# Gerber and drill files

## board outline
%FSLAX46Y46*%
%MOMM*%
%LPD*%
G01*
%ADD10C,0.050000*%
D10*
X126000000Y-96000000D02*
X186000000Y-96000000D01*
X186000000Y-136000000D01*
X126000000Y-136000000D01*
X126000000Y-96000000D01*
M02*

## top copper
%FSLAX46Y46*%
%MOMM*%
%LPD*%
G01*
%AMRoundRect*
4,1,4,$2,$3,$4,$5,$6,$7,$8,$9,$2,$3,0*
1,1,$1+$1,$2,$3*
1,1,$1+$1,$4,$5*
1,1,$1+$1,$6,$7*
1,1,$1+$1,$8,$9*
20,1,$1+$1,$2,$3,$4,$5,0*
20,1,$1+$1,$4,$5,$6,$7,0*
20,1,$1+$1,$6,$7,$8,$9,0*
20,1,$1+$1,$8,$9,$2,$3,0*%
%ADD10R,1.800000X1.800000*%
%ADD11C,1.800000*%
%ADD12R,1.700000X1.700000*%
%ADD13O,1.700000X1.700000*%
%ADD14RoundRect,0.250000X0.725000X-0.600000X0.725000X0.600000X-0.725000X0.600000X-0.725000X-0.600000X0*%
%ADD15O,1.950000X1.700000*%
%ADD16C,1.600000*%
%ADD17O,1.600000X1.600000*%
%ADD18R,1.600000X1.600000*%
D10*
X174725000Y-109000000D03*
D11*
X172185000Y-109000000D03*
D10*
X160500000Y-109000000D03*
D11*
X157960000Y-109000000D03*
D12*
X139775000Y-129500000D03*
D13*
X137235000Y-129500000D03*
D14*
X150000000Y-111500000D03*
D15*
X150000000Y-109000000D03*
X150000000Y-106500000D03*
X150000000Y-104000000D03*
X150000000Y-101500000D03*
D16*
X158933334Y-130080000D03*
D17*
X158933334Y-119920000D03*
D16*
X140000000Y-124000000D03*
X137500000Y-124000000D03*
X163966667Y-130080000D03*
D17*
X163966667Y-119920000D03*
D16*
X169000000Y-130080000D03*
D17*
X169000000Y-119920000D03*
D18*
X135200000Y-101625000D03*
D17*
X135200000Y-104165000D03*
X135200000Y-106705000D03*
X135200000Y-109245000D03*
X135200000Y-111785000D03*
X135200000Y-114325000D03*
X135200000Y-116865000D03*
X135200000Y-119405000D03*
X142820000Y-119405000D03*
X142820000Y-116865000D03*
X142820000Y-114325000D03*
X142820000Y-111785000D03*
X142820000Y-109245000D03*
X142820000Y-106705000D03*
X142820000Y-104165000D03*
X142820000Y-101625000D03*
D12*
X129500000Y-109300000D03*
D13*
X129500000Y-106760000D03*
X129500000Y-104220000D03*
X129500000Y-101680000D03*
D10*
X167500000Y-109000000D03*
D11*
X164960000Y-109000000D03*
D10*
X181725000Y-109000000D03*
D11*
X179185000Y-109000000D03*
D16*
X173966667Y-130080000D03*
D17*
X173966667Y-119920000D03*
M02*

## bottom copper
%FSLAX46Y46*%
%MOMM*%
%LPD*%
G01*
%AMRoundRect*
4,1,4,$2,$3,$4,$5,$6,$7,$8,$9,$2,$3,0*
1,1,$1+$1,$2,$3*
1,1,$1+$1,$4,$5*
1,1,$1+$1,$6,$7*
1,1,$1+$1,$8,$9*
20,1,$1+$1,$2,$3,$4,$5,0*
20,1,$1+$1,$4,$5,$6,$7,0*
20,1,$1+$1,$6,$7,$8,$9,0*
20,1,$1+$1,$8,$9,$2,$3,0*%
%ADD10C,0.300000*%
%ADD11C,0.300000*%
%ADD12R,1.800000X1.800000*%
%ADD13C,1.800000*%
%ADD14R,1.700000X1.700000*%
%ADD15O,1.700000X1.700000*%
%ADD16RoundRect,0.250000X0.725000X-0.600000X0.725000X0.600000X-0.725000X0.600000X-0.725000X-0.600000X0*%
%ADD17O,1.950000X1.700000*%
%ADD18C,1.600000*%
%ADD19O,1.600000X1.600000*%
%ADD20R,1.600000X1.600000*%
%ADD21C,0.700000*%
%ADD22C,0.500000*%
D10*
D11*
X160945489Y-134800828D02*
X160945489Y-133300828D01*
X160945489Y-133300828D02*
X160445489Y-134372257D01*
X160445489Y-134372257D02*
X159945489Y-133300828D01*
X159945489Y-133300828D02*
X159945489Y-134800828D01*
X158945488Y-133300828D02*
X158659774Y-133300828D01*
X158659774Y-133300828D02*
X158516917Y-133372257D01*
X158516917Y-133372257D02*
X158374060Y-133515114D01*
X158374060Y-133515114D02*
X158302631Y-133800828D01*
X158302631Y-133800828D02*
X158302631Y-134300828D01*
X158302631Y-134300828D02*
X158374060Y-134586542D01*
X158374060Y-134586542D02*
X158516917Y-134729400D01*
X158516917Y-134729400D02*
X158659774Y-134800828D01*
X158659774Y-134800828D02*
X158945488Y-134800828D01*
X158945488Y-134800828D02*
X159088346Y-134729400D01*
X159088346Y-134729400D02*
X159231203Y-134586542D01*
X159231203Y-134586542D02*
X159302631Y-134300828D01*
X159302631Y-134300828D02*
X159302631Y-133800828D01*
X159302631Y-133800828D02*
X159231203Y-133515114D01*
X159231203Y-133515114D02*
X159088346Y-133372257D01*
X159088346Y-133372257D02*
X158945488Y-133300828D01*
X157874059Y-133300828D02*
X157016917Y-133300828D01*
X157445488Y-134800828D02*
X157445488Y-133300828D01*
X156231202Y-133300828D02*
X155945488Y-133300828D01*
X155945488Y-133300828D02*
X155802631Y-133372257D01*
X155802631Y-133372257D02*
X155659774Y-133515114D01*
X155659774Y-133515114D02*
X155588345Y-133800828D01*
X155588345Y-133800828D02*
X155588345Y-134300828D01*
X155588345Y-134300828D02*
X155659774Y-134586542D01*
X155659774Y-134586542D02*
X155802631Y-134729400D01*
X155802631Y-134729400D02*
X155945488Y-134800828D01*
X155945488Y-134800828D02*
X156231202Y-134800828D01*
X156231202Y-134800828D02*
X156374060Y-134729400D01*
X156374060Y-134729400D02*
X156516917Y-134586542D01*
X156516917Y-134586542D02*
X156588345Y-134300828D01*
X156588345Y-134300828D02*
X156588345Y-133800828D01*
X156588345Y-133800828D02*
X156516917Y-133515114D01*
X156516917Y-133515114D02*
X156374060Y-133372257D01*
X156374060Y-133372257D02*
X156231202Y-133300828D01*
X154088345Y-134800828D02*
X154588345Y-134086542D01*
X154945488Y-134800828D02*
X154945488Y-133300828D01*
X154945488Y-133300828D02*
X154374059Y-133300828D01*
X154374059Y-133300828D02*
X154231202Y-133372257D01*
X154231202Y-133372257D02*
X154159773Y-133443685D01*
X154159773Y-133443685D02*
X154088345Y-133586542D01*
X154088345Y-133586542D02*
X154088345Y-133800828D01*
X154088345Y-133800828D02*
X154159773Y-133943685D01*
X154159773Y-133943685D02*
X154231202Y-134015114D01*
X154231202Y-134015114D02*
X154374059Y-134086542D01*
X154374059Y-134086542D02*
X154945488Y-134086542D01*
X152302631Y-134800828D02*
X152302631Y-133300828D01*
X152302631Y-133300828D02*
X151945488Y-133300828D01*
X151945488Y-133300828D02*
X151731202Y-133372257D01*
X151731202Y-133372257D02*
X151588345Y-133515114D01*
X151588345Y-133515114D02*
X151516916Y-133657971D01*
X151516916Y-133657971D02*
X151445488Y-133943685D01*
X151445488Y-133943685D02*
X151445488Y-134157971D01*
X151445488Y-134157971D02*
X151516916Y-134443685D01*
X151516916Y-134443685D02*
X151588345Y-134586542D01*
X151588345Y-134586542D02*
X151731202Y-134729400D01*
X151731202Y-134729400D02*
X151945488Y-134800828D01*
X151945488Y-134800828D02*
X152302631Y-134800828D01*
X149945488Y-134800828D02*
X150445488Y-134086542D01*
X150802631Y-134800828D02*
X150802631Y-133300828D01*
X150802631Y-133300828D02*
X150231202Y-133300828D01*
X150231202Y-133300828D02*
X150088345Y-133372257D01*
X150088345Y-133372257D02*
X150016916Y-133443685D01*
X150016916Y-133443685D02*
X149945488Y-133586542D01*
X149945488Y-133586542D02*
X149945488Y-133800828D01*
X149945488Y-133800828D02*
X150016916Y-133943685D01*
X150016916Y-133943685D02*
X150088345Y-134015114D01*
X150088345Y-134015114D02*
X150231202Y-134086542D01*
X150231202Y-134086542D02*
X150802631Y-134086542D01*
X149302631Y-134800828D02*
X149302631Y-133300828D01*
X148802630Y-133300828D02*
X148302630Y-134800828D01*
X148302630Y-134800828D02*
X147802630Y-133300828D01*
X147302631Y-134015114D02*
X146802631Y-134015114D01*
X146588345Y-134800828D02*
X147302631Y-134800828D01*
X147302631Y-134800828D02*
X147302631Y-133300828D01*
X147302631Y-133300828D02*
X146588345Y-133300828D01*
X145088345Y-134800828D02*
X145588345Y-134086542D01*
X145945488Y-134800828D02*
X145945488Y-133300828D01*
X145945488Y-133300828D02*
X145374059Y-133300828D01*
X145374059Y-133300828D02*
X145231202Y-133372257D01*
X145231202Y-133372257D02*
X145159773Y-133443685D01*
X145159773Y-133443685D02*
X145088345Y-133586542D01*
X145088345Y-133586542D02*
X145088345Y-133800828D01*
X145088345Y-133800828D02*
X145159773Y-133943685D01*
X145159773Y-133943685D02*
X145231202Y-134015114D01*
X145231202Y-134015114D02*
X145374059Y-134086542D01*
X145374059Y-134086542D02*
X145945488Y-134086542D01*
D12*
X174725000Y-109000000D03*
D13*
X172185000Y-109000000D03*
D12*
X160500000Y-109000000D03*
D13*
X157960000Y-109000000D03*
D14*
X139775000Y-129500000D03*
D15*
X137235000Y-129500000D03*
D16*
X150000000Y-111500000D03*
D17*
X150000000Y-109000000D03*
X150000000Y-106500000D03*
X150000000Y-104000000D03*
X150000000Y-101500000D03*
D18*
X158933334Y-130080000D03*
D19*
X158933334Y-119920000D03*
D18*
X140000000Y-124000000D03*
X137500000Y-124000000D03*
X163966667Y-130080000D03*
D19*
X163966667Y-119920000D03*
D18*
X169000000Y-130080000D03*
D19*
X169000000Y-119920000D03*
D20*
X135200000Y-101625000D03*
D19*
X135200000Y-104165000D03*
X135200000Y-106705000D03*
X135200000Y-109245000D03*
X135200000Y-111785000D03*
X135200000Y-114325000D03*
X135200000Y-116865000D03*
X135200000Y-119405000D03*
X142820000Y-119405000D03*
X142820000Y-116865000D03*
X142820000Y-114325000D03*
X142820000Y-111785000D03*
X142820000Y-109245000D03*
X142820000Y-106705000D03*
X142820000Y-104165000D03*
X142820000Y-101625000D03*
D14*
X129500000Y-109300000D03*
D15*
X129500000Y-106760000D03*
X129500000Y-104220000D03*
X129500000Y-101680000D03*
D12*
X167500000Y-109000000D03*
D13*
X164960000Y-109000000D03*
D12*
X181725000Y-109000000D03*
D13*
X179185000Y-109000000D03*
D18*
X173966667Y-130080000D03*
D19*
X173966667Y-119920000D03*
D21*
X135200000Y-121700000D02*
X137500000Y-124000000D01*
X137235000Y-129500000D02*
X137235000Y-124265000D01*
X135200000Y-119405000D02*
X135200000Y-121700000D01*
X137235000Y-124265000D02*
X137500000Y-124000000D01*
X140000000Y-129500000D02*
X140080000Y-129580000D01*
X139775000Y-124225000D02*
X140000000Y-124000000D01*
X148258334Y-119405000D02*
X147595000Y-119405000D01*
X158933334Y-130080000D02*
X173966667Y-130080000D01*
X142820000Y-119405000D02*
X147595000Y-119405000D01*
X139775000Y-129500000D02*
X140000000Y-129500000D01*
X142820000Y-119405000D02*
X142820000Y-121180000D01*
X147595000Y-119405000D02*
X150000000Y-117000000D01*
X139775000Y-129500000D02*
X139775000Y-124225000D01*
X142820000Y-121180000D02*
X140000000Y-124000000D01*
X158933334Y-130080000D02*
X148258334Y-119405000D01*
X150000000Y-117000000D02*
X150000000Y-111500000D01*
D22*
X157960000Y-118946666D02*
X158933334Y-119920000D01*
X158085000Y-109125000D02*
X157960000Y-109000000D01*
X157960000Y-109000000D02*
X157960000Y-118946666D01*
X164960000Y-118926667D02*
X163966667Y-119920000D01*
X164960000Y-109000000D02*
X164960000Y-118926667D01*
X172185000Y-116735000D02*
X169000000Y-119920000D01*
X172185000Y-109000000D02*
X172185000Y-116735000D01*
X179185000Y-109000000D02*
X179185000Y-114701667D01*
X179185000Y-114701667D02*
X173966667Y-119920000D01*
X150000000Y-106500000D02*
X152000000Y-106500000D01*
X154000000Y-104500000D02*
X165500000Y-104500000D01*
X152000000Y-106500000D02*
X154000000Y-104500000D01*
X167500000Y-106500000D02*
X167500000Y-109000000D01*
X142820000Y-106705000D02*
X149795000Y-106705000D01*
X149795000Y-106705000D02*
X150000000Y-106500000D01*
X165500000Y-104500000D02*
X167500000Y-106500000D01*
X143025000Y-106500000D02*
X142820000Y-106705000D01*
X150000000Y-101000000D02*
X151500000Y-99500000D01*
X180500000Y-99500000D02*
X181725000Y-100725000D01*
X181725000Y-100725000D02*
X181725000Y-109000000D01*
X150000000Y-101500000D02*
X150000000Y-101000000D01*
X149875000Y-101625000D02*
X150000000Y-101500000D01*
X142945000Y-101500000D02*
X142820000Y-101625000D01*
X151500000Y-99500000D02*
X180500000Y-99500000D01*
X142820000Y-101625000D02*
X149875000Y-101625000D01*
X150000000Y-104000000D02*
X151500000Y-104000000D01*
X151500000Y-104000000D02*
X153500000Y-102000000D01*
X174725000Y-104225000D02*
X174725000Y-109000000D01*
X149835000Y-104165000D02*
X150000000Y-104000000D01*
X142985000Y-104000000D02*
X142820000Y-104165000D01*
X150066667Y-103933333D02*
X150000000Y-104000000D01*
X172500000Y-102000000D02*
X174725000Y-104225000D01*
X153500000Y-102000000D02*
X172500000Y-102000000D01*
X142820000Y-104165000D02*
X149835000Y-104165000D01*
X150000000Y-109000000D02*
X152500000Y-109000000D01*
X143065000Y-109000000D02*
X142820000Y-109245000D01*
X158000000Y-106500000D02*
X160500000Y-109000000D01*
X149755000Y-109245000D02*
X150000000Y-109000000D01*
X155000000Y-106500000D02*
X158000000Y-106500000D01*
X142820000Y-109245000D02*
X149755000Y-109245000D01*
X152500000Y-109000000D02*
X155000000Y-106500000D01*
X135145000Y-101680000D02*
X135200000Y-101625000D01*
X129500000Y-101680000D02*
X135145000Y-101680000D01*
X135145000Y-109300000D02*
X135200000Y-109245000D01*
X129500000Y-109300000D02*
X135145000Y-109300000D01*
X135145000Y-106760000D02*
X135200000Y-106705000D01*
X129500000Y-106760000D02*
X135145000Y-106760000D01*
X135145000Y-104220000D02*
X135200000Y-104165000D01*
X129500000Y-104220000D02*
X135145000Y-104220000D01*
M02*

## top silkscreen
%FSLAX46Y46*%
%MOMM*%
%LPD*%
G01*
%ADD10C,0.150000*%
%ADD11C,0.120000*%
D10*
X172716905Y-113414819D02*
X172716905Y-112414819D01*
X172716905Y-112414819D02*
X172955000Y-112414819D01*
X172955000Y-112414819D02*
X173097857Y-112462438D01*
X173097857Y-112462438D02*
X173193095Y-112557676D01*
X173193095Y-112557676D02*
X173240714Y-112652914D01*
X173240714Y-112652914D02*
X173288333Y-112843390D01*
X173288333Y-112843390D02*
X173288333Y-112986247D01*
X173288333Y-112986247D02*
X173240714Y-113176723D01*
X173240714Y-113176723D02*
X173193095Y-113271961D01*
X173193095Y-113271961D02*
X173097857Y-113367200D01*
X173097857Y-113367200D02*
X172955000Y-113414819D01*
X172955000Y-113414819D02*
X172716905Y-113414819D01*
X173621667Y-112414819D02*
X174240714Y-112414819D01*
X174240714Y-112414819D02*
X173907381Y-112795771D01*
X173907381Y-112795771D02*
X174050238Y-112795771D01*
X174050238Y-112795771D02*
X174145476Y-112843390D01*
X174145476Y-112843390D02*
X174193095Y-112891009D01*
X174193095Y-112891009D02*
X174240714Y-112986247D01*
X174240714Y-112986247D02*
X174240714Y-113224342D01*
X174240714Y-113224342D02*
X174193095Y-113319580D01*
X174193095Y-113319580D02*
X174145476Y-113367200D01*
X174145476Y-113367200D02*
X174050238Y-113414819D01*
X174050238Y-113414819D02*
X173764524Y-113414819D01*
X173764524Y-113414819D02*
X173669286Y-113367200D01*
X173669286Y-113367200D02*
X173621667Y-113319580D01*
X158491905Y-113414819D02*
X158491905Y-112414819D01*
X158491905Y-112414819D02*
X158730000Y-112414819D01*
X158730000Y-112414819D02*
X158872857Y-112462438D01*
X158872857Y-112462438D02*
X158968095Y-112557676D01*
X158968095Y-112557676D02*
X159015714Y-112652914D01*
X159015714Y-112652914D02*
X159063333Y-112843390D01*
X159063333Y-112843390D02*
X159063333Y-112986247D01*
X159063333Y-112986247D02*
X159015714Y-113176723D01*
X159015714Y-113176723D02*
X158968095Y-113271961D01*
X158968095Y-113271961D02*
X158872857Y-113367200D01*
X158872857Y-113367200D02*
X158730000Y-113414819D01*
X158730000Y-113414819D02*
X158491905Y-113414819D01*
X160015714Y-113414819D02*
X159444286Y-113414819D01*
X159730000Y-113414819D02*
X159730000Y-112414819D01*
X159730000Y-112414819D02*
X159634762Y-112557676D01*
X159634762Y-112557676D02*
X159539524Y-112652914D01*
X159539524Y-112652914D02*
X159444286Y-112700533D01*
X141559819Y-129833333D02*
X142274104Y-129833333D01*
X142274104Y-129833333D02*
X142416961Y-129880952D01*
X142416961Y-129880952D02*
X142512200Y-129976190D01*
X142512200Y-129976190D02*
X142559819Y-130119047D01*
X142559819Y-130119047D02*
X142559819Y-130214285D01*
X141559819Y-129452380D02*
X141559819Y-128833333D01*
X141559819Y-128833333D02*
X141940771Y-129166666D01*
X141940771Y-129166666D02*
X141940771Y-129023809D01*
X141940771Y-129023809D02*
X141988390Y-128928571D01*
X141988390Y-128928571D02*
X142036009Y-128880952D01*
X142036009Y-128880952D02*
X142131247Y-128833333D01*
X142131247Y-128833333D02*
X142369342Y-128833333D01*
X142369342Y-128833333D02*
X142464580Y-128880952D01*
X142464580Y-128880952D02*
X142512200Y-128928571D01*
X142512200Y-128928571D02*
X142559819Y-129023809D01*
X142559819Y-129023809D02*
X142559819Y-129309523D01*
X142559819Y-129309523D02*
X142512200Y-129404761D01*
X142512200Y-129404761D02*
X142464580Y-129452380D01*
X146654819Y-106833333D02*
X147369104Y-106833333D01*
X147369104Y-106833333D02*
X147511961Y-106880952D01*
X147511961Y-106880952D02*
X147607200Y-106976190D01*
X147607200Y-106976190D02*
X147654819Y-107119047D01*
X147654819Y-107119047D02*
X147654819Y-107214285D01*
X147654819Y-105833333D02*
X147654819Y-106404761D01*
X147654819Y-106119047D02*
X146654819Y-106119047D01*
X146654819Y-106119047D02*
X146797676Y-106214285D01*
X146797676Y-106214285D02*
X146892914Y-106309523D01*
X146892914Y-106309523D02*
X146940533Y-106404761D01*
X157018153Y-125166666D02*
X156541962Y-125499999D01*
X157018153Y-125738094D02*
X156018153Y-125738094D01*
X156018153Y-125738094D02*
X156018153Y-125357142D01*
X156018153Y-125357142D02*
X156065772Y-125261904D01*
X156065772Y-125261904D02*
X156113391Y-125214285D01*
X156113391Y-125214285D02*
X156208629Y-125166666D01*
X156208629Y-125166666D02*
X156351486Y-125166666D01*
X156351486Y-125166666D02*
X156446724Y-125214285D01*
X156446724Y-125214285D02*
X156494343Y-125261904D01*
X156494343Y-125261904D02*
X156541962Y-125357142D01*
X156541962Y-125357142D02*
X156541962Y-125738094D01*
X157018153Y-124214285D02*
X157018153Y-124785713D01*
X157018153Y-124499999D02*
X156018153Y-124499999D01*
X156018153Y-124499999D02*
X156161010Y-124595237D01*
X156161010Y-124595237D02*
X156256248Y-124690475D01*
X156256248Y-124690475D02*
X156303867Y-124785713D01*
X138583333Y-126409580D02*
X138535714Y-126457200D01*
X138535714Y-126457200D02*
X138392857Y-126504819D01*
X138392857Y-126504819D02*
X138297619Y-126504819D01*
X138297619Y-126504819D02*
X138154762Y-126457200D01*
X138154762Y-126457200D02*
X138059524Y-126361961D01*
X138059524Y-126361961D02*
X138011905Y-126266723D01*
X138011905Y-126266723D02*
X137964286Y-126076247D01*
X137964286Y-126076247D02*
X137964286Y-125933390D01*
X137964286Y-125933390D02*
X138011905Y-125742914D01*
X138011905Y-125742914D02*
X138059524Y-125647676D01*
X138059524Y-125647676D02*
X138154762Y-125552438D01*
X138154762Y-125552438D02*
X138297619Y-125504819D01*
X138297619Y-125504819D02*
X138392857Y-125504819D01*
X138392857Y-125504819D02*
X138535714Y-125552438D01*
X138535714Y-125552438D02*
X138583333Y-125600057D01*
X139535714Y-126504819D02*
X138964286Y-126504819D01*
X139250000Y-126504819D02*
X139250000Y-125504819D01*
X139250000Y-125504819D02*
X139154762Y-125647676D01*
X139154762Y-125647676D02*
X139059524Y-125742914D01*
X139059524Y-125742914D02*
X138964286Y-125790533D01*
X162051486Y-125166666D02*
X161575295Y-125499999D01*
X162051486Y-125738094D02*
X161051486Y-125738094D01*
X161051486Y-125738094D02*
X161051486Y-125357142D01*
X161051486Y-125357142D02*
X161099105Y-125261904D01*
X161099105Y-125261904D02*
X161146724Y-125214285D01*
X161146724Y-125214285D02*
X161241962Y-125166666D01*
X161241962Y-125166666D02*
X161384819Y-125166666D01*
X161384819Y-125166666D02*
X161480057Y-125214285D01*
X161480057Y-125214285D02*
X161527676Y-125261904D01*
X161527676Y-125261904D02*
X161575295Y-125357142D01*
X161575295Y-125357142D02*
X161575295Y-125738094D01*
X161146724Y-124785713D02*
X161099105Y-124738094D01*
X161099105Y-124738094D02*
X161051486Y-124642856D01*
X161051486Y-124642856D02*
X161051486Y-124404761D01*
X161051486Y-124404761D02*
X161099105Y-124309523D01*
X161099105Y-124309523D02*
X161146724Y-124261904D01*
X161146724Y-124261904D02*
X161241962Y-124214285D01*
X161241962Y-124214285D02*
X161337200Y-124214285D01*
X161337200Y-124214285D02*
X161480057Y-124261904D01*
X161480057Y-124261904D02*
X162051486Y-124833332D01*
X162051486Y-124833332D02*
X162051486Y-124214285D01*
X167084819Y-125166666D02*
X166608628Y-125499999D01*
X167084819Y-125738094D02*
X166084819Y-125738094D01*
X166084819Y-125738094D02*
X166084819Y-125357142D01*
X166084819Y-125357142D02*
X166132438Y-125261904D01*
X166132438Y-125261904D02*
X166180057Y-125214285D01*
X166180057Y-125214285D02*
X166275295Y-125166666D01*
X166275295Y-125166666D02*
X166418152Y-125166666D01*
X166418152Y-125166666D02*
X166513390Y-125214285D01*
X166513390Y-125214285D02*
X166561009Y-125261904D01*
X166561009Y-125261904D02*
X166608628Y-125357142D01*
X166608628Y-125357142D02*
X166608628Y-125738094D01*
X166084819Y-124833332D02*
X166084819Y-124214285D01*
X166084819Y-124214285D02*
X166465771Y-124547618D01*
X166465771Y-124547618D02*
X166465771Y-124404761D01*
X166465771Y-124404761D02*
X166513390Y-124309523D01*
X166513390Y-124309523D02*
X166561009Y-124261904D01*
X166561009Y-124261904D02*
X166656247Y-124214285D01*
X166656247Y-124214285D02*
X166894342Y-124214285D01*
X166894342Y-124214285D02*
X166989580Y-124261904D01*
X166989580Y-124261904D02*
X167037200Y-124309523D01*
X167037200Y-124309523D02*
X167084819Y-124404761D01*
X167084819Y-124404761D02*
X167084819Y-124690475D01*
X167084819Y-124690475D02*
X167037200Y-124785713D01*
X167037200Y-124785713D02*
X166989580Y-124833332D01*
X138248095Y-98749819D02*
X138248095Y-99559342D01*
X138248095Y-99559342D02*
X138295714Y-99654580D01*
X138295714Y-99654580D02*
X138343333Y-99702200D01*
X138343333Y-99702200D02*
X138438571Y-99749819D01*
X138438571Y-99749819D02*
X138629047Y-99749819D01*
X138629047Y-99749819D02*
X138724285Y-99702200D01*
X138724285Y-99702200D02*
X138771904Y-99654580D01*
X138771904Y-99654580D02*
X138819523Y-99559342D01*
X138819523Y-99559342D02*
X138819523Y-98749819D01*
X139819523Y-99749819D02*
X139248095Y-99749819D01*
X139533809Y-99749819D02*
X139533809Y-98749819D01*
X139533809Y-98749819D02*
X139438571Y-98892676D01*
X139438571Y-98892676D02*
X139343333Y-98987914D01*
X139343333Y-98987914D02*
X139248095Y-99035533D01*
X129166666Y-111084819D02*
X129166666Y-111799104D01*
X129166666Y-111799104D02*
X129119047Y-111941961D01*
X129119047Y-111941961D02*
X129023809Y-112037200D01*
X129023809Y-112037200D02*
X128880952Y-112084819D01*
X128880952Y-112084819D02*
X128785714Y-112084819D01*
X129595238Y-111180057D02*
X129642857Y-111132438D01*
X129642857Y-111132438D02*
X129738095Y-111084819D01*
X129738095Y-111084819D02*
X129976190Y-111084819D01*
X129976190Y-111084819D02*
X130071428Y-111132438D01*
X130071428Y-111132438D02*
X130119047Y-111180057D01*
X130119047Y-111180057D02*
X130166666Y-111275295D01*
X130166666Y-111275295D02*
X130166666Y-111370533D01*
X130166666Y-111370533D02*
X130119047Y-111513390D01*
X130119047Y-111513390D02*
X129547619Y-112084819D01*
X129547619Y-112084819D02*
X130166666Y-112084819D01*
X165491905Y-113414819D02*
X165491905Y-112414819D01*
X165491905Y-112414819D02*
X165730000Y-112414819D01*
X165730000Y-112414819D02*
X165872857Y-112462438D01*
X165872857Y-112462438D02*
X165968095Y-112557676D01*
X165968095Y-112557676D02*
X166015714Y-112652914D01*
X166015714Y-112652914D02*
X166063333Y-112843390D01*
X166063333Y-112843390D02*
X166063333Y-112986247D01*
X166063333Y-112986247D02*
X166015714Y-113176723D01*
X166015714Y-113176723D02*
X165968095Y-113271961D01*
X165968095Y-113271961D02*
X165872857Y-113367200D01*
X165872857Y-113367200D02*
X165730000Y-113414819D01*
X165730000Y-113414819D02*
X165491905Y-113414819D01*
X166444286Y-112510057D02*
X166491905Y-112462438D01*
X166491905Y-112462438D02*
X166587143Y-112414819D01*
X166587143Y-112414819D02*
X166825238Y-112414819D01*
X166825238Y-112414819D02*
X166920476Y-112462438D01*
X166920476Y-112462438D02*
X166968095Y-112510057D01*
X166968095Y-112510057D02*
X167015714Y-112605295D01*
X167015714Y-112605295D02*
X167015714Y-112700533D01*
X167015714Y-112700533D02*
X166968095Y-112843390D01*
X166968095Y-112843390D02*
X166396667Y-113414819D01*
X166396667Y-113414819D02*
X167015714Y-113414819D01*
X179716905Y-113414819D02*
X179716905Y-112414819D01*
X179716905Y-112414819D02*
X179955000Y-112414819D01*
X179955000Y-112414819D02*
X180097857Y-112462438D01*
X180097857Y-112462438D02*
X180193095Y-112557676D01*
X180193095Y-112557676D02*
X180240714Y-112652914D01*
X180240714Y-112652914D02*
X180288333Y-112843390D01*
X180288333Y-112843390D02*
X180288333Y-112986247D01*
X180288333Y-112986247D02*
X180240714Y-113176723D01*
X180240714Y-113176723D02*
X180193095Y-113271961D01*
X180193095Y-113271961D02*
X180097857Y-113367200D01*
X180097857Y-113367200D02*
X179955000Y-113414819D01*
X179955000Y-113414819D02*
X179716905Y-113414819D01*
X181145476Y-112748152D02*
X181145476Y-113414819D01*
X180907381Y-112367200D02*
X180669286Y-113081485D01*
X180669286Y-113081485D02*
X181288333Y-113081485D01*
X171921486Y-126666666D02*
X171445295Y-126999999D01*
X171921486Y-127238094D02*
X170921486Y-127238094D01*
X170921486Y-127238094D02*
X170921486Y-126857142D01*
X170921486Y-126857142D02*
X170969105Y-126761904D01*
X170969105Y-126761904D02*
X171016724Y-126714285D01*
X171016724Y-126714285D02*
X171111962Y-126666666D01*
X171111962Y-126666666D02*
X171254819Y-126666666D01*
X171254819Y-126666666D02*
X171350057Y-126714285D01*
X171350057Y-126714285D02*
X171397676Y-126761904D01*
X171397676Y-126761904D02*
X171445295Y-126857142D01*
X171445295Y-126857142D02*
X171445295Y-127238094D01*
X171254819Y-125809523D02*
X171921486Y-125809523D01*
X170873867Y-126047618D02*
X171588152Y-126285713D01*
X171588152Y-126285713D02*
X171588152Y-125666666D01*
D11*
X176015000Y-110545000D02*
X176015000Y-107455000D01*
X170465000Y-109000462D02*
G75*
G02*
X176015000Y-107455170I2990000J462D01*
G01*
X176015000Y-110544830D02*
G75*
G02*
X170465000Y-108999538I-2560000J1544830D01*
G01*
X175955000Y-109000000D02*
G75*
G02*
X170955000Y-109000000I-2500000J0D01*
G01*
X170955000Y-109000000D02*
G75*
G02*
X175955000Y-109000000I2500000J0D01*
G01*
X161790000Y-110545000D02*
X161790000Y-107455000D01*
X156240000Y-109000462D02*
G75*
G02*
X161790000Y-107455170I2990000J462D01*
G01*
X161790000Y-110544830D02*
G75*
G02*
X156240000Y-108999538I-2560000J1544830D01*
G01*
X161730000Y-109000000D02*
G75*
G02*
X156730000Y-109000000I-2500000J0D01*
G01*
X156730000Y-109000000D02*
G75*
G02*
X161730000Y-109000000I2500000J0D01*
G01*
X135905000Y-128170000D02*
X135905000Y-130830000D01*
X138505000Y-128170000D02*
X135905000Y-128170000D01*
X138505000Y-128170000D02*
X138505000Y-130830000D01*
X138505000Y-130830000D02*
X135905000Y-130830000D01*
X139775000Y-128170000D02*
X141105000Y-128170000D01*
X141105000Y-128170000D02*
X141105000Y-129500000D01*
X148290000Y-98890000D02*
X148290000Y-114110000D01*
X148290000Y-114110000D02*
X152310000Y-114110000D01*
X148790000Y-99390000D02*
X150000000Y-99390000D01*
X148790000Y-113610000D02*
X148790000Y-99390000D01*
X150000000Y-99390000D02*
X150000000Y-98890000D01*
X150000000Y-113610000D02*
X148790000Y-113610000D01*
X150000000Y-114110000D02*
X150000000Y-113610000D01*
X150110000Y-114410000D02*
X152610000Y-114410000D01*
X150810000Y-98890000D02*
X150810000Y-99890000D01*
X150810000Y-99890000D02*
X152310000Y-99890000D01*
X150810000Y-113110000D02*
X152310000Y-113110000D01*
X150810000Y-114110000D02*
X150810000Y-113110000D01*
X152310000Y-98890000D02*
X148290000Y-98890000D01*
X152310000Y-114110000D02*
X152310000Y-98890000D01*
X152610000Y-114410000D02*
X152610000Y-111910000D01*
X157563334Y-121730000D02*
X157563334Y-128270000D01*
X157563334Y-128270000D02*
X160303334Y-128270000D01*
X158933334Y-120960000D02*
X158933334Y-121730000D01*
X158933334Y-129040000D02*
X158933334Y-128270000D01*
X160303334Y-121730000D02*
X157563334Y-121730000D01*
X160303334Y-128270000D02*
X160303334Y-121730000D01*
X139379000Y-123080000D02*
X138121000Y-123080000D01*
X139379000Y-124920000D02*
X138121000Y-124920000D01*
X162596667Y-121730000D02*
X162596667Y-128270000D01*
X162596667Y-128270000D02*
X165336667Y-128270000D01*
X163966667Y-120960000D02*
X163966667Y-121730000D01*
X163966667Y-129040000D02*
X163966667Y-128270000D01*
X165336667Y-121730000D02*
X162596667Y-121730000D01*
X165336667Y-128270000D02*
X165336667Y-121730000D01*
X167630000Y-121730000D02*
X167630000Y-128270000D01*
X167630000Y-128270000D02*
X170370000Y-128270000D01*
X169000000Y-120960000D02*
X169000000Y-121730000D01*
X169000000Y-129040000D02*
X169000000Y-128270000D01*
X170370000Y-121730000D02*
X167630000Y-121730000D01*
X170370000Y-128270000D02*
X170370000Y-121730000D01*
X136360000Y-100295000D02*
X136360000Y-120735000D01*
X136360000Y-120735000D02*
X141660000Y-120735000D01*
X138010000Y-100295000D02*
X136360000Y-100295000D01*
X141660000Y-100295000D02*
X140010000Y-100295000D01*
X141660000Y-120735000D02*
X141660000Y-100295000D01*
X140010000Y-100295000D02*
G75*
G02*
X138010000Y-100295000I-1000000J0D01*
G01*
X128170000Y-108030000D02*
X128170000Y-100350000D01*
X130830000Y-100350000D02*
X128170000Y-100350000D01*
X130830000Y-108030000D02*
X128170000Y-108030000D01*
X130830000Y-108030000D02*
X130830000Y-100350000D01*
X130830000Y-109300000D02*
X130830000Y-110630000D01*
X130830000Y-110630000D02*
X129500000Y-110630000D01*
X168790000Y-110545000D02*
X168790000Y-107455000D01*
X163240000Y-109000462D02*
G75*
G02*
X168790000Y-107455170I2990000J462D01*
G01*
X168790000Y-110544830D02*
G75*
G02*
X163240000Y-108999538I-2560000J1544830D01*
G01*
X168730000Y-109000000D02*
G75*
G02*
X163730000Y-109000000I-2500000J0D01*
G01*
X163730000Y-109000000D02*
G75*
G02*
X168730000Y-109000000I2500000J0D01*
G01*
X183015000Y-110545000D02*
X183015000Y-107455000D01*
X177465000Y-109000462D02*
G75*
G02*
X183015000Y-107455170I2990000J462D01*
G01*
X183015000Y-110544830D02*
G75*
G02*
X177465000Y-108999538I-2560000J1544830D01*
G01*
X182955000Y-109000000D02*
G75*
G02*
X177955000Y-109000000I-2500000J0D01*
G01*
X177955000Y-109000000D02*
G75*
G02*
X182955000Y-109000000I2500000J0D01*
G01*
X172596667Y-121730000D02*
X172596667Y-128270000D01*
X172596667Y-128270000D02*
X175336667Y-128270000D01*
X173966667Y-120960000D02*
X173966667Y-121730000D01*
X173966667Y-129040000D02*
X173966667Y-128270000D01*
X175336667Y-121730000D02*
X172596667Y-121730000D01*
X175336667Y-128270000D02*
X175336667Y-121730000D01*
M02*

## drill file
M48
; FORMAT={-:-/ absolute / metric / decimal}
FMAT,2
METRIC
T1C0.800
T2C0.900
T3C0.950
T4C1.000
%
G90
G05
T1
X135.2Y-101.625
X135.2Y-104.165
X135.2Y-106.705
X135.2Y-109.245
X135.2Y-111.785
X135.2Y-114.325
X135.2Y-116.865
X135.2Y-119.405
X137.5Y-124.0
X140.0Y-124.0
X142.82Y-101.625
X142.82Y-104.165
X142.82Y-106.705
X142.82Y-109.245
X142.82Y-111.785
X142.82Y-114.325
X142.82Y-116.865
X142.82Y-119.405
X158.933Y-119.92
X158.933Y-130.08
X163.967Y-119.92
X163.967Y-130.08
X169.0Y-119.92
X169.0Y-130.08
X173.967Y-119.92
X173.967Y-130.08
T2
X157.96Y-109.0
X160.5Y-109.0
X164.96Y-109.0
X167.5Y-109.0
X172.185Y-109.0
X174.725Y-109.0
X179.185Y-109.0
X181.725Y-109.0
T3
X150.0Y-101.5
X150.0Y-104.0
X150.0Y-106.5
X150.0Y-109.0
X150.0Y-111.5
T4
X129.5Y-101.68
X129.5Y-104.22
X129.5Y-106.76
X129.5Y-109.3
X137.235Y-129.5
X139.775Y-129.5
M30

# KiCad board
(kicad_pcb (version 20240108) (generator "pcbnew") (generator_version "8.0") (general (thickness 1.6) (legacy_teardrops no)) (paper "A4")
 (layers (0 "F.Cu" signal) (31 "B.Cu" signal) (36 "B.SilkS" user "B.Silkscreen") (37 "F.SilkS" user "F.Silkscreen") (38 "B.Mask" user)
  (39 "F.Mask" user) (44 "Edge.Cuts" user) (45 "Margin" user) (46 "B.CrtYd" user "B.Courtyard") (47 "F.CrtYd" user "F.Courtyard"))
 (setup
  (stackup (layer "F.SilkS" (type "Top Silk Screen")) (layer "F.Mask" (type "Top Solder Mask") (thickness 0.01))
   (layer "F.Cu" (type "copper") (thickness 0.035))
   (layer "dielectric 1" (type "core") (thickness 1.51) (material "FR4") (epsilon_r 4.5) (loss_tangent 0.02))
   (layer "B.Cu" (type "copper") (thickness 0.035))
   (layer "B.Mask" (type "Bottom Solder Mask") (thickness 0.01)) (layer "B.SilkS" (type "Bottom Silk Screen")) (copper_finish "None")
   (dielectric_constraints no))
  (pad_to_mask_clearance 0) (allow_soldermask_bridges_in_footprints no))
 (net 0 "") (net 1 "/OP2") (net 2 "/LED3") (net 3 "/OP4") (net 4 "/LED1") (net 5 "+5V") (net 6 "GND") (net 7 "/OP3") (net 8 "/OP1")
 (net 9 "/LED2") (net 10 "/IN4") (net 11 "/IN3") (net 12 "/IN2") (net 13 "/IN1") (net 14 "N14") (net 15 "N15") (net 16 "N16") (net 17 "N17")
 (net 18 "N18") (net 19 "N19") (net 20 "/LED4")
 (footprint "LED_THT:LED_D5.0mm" (layer "F.Cu") (at 174.725 109 180)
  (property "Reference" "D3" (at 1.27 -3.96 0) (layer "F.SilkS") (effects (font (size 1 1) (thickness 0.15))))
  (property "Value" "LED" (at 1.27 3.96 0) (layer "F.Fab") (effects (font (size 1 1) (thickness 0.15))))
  (fp_line (start -1.29 -1.545) (end -1.29 1.545) (stroke (width 0.12) (type solid)) (layer "F.SilkS"))
  (fp_arc (start 4.26 -0.000462) (mid 2.072002 2.880433) (end -1.29 1.54483) (stroke (width 0.12) (type solid)) (layer "F.SilkS"))
  (fp_arc (start -1.29 -1.54483) (mid 2.072002 -2.880433) (end 4.26 0.000462) (stroke (width 0.12) (type solid)) (layer "F.SilkS"))
  (fp_circle (center 1.27 0) (end 3.77 0) (stroke (width 0.12) (type solid)) (fill none) (layer "F.SilkS"))
  (pad "1" thru_hole rect (at 0 0 180) (size 1.8 1.8) (drill 0.9) (layers "*.Cu" "*.Mask") (remove_unused_layers no) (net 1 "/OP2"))
  (pad "2" thru_hole circle (at 2.54 0 180) (size 1.8 1.8) (drill 0.9) (layers "*.Cu" "*.Mask") (remove_unused_layers no) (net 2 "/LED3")))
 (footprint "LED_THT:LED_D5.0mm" (layer "F.Cu") (at 160.5 109 180)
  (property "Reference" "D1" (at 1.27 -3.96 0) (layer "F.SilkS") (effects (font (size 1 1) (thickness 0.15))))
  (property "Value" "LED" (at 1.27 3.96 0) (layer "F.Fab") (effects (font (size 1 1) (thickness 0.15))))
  (fp_line (start -1.29 -1.545) (end -1.29 1.545) (stroke (width 0.12) (type solid)) (layer "F.SilkS"))
  (fp_arc (start 4.26 -0.000462) (mid 2.072002 2.880433) (end -1.29 1.54483) (stroke (width 0.12) (type solid)) (layer "F.SilkS"))
  (fp_arc (start -1.29 -1.54483) (mid 2.072002 -2.880433) (end 4.26 0.000462) (stroke (width 0.12) (type solid)) (layer "F.SilkS"))
  (fp_circle (center 1.27 0) (end 3.77 0) (stroke (width 0.12) (type solid)) (fill none) (layer "F.SilkS"))
  (pad "1" thru_hole rect (at 0 0 180) (size 1.8 1.8) (drill 0.9) (layers "*.Cu" "*.Mask") (remove_unused_layers no) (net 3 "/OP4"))
  (pad "2" thru_hole circle (at 2.54 0 180) (size 1.8 1.8) (drill 0.9) (layers "*.Cu" "*.Mask") (remove_unused_layers no) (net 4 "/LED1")))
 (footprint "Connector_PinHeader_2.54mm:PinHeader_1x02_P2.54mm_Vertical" (layer "F.Cu") (at 139.775 129.5 -90)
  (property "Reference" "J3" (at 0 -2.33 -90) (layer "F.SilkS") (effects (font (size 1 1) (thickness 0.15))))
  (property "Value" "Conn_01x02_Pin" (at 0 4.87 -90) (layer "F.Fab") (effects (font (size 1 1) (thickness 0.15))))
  (fp_line (start -1.33 3.87) (end 1.33 3.87) (stroke (width 0.12) (type solid)) (layer "F.SilkS"))
  (fp_line (start -1.33 1.27) (end -1.33 3.87) (stroke (width 0.12) (type solid)) (layer "F.SilkS"))
  (fp_line (start -1.33 1.27) (end 1.33 1.27) (stroke (width 0.12) (type solid)) (layer "F.SilkS"))
  (fp_line (start 1.33 1.27) (end 1.33 3.87) (stroke (width 0.12) (type solid)) (layer "F.SilkS"))
  (fp_line (start -1.33 0) (end -1.33 -1.33) (stroke (width 0.12) (type solid)) (layer "F.SilkS"))
  (fp_line (start -1.33 -1.33) (end 0 -1.33) (stroke (width 0.12) (type solid)) (layer "F.SilkS"))
  (pad "1" thru_hole rect (at 0 0 270) (size 1.7 1.7) (drill 1) (layers "*.Cu" "*.Mask") (remove_unused_layers no) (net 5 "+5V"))
  (pad "2" thru_hole oval (at 0 2.54 270) (size 1.7 1.7) (drill 1) (layers "*.Cu" "*.Mask") (remove_unused_layers no) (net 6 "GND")))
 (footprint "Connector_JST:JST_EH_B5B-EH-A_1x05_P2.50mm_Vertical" (layer "F.Cu") (at 150 111.5 90)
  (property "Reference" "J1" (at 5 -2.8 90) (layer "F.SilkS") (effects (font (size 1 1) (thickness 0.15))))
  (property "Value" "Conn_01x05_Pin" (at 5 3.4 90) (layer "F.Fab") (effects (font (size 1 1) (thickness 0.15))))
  (fp_line (start 12.61 -1.71) (end -2.61 -1.71) (stroke (width 0.12) (type solid)) (layer "F.SilkS"))
  (fp_line (start -2.61 -1.71) (end -2.61 2.31) (stroke (width 0.12) (type solid)) (layer "F.SilkS"))
  (fp_line (start 12.11 -1.21) (end 12.11 0) (stroke (width 0.12) (type solid)) (layer "F.SilkS"))
  (fp_line (start -2.11 -1.21) (end 12.11 -1.21) (stroke (width 0.12) (type solid)) (layer "F.SilkS"))
  (fp_line (start 12.11 0) (end 12.61 0) (stroke (width 0.12) (type solid)) (layer "F.SilkS"))
  (fp_line (start -2.11 0) (end -2.11 -1.21) (stroke (width 0.12) (type solid)) (layer "F.SilkS"))
  (fp_line (start -2.61 0) (end -2.11 0) (stroke (width 0.12) (type solid)) (layer "F.SilkS"))
  (fp_line (start -2.91 0.11) (end -2.91 2.61) (stroke (width 0.12) (type solid)) (layer "F.SilkS"))
  (fp_line (start 12.61 0.81) (end 11.61 0.81) (stroke (width 0.12) (type solid)) (layer "F.SilkS"))
  (fp_line (start 11.61 0.81) (end 11.61 2.31) (stroke (width 0.12) (type solid)) (layer "F.SilkS"))
  (fp_line (start -1.61 0.81) (end -1.61 2.31) (stroke (width 0.12) (type solid)) (layer "F.SilkS"))
  (fp_line (start -2.61 0.81) (end -1.61 0.81) (stroke (width 0.12) (type solid)) (layer "F.SilkS"))
  (fp_line (start 12.61 2.31) (end 12.61 -1.71) (stroke (width 0.12) (type solid)) (layer "F.SilkS"))
  (fp_line (start -2.61 2.31) (end 12.61 2.31) (stroke (width 0.12) (type solid)) (layer "F.SilkS"))
  (fp_line (start -2.91 2.61) (end -0.41 2.61) (stroke (width 0.12) (type solid)) (layer "F.SilkS"))
  (pad "1" thru_hole roundrect (at 0 0 90) (size 1.7 1.95) (drill 0.95) (layers "*.Cu" "*.Mask") (remove_unused_layers no)
   (roundrect_rratio 0.147059) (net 5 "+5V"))
  (pad "2" thru_hole oval (at 2.5 0 90) (size 1.7 1.95) (drill 0.95) (layers "*.Cu" "*.Mask") (remove_unused_layers no) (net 3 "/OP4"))
  (pad "3" thru_hole oval (at 5 0 90) (size 1.7 1.95) (drill 0.95) (layers "*.Cu" "*.Mask") (remove_unused_layers no) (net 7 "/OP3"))
  (pad "4" thru_hole oval (at 7.5 0 90) (size 1.7 1.95) (drill 0.95) (layers "*.Cu" "*.Mask") (remove_unused_layers no) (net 1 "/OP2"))
  (pad "5" thru_hole oval (at 10 0 90) (size 1.7 1.95) (drill 0.95) (layers "*.Cu" "*.Mask") (remove_unused_layers no) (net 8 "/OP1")))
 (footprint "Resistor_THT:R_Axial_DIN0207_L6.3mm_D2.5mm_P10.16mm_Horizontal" (layer "F.Cu") (at 158.933334 130.08 90)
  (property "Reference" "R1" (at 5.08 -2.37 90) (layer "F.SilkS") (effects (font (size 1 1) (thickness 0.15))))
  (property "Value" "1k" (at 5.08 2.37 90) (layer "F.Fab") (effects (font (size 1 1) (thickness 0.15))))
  (fp_line (start 8.35 -1.37) (end 1.81 -1.37) (stroke (width 0.12) (type solid)) (layer "F.SilkS"))
  (fp_line (start 1.81 -1.37) (end 1.81 1.37) (stroke (width 0.12) (type solid)) (layer "F.SilkS"))
  (fp_line (start 9.12 0) (end 8.35 0) (stroke (width 0.12) (type solid)) (layer "F.SilkS"))
  (fp_line (start 1.04 0) (end 1.81 0) (stroke (width 0.12) (type solid)) (layer "F.SilkS"))
  (fp_line (start 8.35 1.37) (end 8.35 -1.37) (stroke (width 0.12) (type solid)) (layer "F.SilkS"))
  (fp_line (start 1.81 1.37) (end 8.35 1.37) (stroke (width 0.12) (type solid)) (layer "F.SilkS"))
  (pad "1" thru_hole circle (at 0 0 90) (size 1.6 1.6) (drill 0.8) (layers "*.Cu" "*.Mask") (remove_unused_layers no) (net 5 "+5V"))
  (pad "2" thru_hole oval (at 10.16 0 90) (size 1.6 1.6) (drill 0.8) (layers "*.Cu" "*.Mask") (remove_unused_layers no) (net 4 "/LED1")))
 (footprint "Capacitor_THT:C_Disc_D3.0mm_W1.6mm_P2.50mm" (layer "F.Cu") (at 140 124 180)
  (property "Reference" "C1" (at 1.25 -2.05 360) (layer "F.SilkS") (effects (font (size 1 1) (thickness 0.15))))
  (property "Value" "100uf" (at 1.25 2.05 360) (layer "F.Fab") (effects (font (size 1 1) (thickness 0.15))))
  (fp_line (start 0.621 0.92) (end 1.879 0.92) (stroke (width 0.12) (type solid)) (layer "F.SilkS"))
  (fp_line (start 0.621 -0.92) (end 1.879 -0.92) (stroke (width 0.12) (type solid)) (layer "F.SilkS"))
  (pad "1" thru_hole circle (at 0 0 180) (size 1.6 1.6) (drill 0.8) (layers "*.Cu" "*.Mask") (remove_unused_layers no) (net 5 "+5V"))
  (pad "2" thru_hole circle (at 2.5 0 180) (size 1.6 1.6) (drill 0.8) (layers "*.Cu" "*.Mask") (remove_unused_layers no) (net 6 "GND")))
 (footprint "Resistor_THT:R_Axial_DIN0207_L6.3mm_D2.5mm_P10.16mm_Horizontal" (layer "F.Cu") (at 163.966667 130.08 90)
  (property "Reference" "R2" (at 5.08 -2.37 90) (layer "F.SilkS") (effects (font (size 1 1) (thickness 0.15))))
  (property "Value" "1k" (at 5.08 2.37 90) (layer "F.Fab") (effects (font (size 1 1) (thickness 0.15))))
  (fp_line (start 8.35 -1.37) (end 1.81 -1.37) (stroke (width 0.12) (type solid)) (layer "F.SilkS"))
  (fp_line (start 1.81 -1.37) (end 1.81 1.37) (stroke (width 0.12) (type solid)) (layer "F.SilkS"))
  (fp_line (start 9.12 0) (end 8.35 0) (stroke (width 0.12) (type solid)) (layer "F.SilkS"))
  (fp_line (start 1.04 0) (end 1.81 0) (stroke (width 0.12) (type solid)) (layer "F.SilkS"))
  (fp_line (start 8.35 1.37) (end 8.35 -1.37) (stroke (width 0.12) (type solid)) (layer "F.SilkS"))
  (fp_line (start 1.81 1.37) (end 8.35 1.37) (stroke (width 0.12) (type solid)) (layer "F.SilkS"))
  (pad "1" thru_hole circle (at 0 0 90) (size 1.6 1.6) (drill 0.8) (layers "*.Cu" "*.Mask") (remove_unused_layers no) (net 5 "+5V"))
  (pad "2" thru_hole oval (at 10.16 0 90) (size 1.6 1.6) (drill 0.8) (layers "*.Cu" "*.Mask") (remove_unused_layers no) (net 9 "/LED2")))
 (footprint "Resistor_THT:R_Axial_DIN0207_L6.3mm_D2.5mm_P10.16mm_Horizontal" (layer "F.Cu") (at 169 130.08 90)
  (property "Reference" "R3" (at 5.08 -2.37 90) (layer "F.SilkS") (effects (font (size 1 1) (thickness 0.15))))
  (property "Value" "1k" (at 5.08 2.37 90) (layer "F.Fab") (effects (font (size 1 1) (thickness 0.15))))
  (fp_line (start 8.35 -1.37) (end 1.81 -1.37) (stroke (width 0.12) (type solid)) (layer "F.SilkS"))
  (fp_line (start 1.81 -1.37) (end 1.81 1.37) (stroke (width 0.12) (type solid)) (layer "F.SilkS"))
  (fp_line (start 9.12 0) (end 8.35 0) (stroke (width 0.12) (type solid)) (layer "F.SilkS"))
  (fp_line (start 1.04 0) (end 1.81 0) (stroke (width 0.12) (type solid)) (layer "F.SilkS"))
  (fp_line (start 8.35 1.37) (end 8.35 -1.37) (stroke (width 0.12) (type solid)) (layer "F.SilkS"))
  (fp_line (start 1.81 1.37) (end 8.35 1.37) (stroke (width 0.12) (type solid)) (layer "F.SilkS"))
  (pad "1" thru_hole circle (at 0 0 90) (size 1.6 1.6) (drill 0.8) (layers "*.Cu" "*.Mask") (remove_unused_layers no) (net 5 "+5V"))
  (pad "2" thru_hole oval (at 10.16 0 90) (size 1.6 1.6) (drill 0.8) (layers "*.Cu" "*.Mask") (remove_unused_layers no) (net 2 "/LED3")))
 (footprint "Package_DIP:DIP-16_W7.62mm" (layer "F.Cu") (at 135.2 101.625)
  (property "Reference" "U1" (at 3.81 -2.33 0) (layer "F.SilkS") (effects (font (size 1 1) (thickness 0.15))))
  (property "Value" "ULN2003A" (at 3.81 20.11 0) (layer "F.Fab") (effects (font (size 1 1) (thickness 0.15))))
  (fp_line (start 1.16 -1.33) (end 1.16 19.11) (stroke (width 0.12) (type solid)) (layer "F.SilkS"))
  (fp_line (start 1.16 19.11) (end 6.46 19.11) (stroke (width 0.12) (type solid)) (layer "F.SilkS"))
  (fp_line (start 2.81 -1.33) (end 1.16 -1.33) (stroke (width 0.12) (type solid)) (layer "F.SilkS"))
  (fp_line (start 6.46 -1.33) (end 4.81 -1.33) (stroke (width 0.12) (type solid)) (layer "F.SilkS"))
  (fp_line (start 6.46 19.11) (end 6.46 -1.33) (stroke (width 0.12) (type solid)) (layer "F.SilkS"))
  (fp_arc (start 4.81 -1.33) (mid 3.81 -0.33) (end 2.81 -1.33) (stroke (width 0.12) (type solid)) (layer "F.SilkS"))
  (pad "1" thru_hole rect (at 0 0) (size 1.6 1.6) (drill 0.8) (layers "*.Cu" "*.Mask") (remove_unused_layers no) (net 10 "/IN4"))
  (pad "2" thru_hole oval (at 0 2.54) (size 1.6 1.6) (drill 0.8) (layers "*.Cu" "*.Mask") (remove_unused_layers no) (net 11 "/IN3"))
  (pad "3" thru_hole oval (at 0 5.08) (size 1.6 1.6) (drill 0.8) (layers "*.Cu" "*.Mask") (remove_unused_layers no) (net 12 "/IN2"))
  (pad "4" thru_hole oval (at 0 7.62) (size 1.6 1.6) (drill 0.8) (layers "*.Cu" "*.Mask") (remove_unused_layers no) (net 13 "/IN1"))
  (pad "5" thru_hole oval (at 0 10.16) (size 1.6 1.6) (drill 0.8) (layers "*.Cu" "*.Mask") (remove_unused_layers no) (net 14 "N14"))
  (pad "6" thru_hole oval (at 0 12.7) (size 1.6 1.6) (drill 0.8) (layers "*.Cu" "*.Mask") (remove_unused_layers no) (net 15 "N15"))
  (pad "7" thru_hole oval (at 0 15.24) (size 1.6 1.6) (drill 0.8) (layers "*.Cu" "*.Mask") (remove_unused_layers no) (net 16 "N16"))
  (pad "8" thru_hole oval (at 0 17.78) (size 1.6 1.6) (drill 0.8) (layers "*.Cu" "*.Mask") (remove_unused_layers no) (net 6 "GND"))
  (pad "9" thru_hole oval (at 7.62 17.78) (size 1.6 1.6) (drill 0.8) (layers "*.Cu" "*.Mask") (remove_unused_layers no) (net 5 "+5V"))
  (pad "10" thru_hole oval (at 7.62 15.24) (size 1.6 1.6) (drill 0.8) (layers "*.Cu" "*.Mask") (remove_unused_layers no) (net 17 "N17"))
  (pad "11" thru_hole oval (at 7.62 12.7) (size 1.6 1.6) (drill 0.8) (layers "*.Cu" "*.Mask") (remove_unused_layers no) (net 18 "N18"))
  (pad "12" thru_hole oval (at 7.62 10.16) (size 1.6 1.6) (drill 0.8) (layers "*.Cu" "*.Mask") (remove_unused_layers no) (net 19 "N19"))
  (pad "13" thru_hole oval (at 7.62 7.62) (size 1.6 1.6) (drill 0.8) (layers "*.Cu" "*.Mask") (remove_unused_layers no) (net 3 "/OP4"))
  (pad "14" thru_hole oval (at 7.62 5.08) (size 1.6 1.6) (drill 0.8) (layers "*.Cu" "*.Mask") (remove_unused_layers no) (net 7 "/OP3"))
  (pad "15" thru_hole oval (at 7.62 2.54) (size 1.6 1.6) (drill 0.8) (layers "*.Cu" "*.Mask") (remove_unused_layers no) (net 1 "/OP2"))
  (pad "16" thru_hole oval (at 7.62 0) (size 1.6 1.6) (drill 0.8) (layers "*.Cu" "*.Mask") (remove_unused_layers no) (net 8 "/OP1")))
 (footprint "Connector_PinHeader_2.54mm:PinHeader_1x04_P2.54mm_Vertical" (layer "F.Cu") (at 129.5 109.3 180)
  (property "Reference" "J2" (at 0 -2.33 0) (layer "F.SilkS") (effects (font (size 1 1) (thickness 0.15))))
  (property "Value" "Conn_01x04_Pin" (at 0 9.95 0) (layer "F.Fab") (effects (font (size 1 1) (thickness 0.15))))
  (fp_line (start 1.33 1.27) (end 1.33 8.95) (stroke (width 0.12) (type solid)) (layer "F.SilkS"))
  (fp_line (start -1.33 8.95) (end 1.33 8.95) (stroke (width 0.12) (type solid)) (layer "F.SilkS"))
  (fp_line (start -1.33 1.27) (end 1.33 1.27) (stroke (width 0.12) (type solid)) (layer "F.SilkS"))
  (fp_line (start -1.33 1.27) (end -1.33 8.95) (stroke (width 0.12) (type solid)) (layer "F.SilkS"))
  (fp_line (start -1.33 0) (end -1.33 -1.33) (stroke (width 0.12) (type solid)) (layer "F.SilkS"))
  (fp_line (start -1.33 -1.33) (end 0 -1.33) (stroke (width 0.12) (type solid)) (layer "F.SilkS"))
  (pad "1" thru_hole rect (at 0 0 180) (size 1.7 1.7) (drill 1) (layers "*.Cu" "*.Mask") (remove_unused_layers no) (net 13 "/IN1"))
  (pad "2" thru_hole oval (at 0 2.54 180) (size 1.7 1.7) (drill 1) (layers "*.Cu" "*.Mask") (remove_unused_layers no) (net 12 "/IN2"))
  (pad "3" thru_hole oval (at 0 5.08 180) (size 1.7 1.7) (drill 1) (layers "*.Cu" "*.Mask") (remove_unused_layers no) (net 11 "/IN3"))
  (pad "4" thru_hole oval (at 0 7.62 180) (size 1.7 1.7) (drill 1) (layers "*.Cu" "*.Mask") (remove_unused_layers no) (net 10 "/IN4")))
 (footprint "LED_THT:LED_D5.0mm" (layer "F.Cu") (at 167.5 109 180)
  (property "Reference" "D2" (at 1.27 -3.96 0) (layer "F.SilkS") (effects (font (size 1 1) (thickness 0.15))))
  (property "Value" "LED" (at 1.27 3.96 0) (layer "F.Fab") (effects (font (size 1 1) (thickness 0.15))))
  (fp_line (start -1.29 -1.545) (end -1.29 1.545) (stroke (width 0.12) (type solid)) (layer "F.SilkS"))
  (fp_arc (start 4.26 -0.000462) (mid 2.072002 2.880433) (end -1.29 1.54483) (stroke (width 0.12) (type solid)) (layer "F.SilkS"))
  (fp_arc (start -1.29 -1.54483) (mid 2.072002 -2.880433) (end 4.26 0.000462) (stroke (width 0.12) (type solid)) (layer "F.SilkS"))
  (fp_circle (center 1.27 0) (end 3.77 0) (stroke (width 0.12) (type solid)) (fill none) (layer "F.SilkS"))
  (pad "1" thru_hole rect (at 0 0 180) (size 1.8 1.8) (drill 0.9) (layers "*.Cu" "*.Mask") (remove_unused_layers no) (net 7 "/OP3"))
  (pad "2" thru_hole circle (at 2.54 0 180) (size 1.8 1.8) (drill 0.9) (layers "*.Cu" "*.Mask") (remove_unused_layers no) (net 9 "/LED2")))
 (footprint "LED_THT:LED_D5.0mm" (layer "F.Cu") (at 181.725 109 180)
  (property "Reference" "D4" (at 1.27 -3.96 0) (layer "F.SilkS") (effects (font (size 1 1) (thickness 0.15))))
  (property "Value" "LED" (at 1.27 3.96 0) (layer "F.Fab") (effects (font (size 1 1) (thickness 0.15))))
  (fp_line (start -1.29 -1.545) (end -1.29 1.545) (stroke (width 0.12) (type solid)) (layer "F.SilkS"))
  (fp_arc (start 4.26 -0.000462) (mid 2.072002 2.880433) (end -1.29 1.54483) (stroke (width 0.12) (type solid)) (layer "F.SilkS"))
  (fp_arc (start -1.29 -1.54483) (mid 2.072002 -2.880433) (end 4.26 0.000462) (stroke (width 0.12) (type solid)) (layer "F.SilkS"))
  (fp_circle (center 1.27 0) (end 3.77 0) (stroke (width 0.12) (type solid)) (fill none) (layer "F.SilkS"))
  (pad "1" thru_hole rect (at 0 0 180) (size 1.8 1.8) (drill 0.9) (layers "*.Cu" "*.Mask") (remove_unused_layers no) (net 8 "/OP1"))
  (pad "2" thru_hole circle (at 2.54 0 180) (size 1.8 1.8) (drill 0.9) (layers "*.Cu" "*.Mask") (remove_unused_layers no) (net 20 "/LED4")))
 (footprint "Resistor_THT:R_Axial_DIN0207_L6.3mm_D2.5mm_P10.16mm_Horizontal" (layer "F.Cu") (at 173.966667 130.08 90)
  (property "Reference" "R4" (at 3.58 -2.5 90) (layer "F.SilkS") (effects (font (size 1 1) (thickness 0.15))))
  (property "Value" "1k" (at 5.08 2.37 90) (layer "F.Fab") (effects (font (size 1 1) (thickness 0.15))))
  (fp_line (start 8.35 -1.37) (end 1.81 -1.37) (stroke (width 0.12) (type solid)) (layer "F.SilkS"))
  (fp_line (start 1.81 -1.37) (end 1.81 1.37) (stroke (width 0.12) (type solid)) (layer "F.SilkS"))
  (fp_line (start 9.12 0) (end 8.35 0) (stroke (width 0.12) (type solid)) (layer "F.SilkS"))
  (fp_line (start 1.04 0) (end 1.81 0) (stroke (width 0.12) (type solid)) (layer "F.SilkS"))
  (fp_line (start 8.35 1.37) (end 8.35 -1.37) (stroke (width 0.12) (type solid)) (layer "F.SilkS"))
  (fp_line (start 1.81 1.37) (end 8.35 1.37) (stroke (width 0.12) (type solid)) (layer "F.SilkS"))
  (pad "1" thru_hole circle (at 0 0 90) (size 1.6 1.6) (drill 0.8) (layers "*.Cu" "*.Mask") (remove_unused_layers no) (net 5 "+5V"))
  (pad "2" thru_hole oval (at 10.16 0 90) (size 1.6 1.6) (drill 0.8) (layers "*.Cu" "*.Mask") (remove_unused_layers no) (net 20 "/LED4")))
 (gr_rect (start 126 96) (end 186 136) (stroke (width 0.05) (type default)) (fill none) (layer "Edge.Cuts"))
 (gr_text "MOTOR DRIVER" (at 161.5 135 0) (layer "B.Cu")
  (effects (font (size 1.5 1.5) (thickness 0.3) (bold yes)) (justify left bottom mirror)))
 (segment (start 135.2 121.7) (end 137.5 124) (width 0.7) (layer "B.Cu") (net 6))
 (segment (start 137.235 129.5) (end 137.235 124.265) (width 0.7) (layer "B.Cu") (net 6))
 (segment (start 135.2 119.405) (end 135.2 121.7) (width 0.7) (layer "B.Cu") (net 6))
 (segment (start 137.235 124.265) (end 137.5 124) (width 0.7) (layer "B.Cu") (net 6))
 (segment (start 140 129.5) (end 140.08 129.58) (width 0.7) (layer "B.Cu") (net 5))
 (segment (start 139.775 124.225) (end 140 124) (width 0.7) (layer "B.Cu") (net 5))
 (segment (start 148.258334 119.405) (end 147.595 119.405) (width 0.7) (layer "B.Cu") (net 5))
 (segment (start 158.933334 130.08) (end 173.966667 130.08) (width 0.7) (layer "B.Cu") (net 5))
 (segment (start 142.82 119.405) (end 147.595 119.405) (width 0.7) (layer "B.Cu") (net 5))
 (segment (start 139.775 129.5) (end 140 129.5) (width 0.7) (layer "B.Cu") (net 5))
 (segment (start 142.82 119.405) (end 142.82 121.18) (width 0.7) (layer "B.Cu") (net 5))
 (segment (start 147.595 119.405) (end 150 117) (width 0.7) (layer "B.Cu") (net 5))
 (segment (start 139.775 129.5) (end 139.775 124.225) (width 0.7) (layer "B.Cu") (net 5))
 (segment (start 142.82 121.18) (end 140 124) (width 0.7) (layer "B.Cu") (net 5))
 (segment (start 158.933334 130.08) (end 148.258334 119.405) (width 0.7) (layer "B.Cu") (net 5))
 (segment (start 150 117) (end 150 111.5) (width 0.7) (layer "B.Cu") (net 5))
 (segment (start 157.96 118.946666) (end 158.933334 119.92) (width 0.5) (layer "B.Cu") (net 4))
 (segment (start 158.085 109.125) (end 157.96 109) (width 0.5) (layer "B.Cu") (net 4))
 (segment (start 157.96 109) (end 157.96 118.946666) (width 0.5) (layer "B.Cu") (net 4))
 (segment (start 164.96 118.926667) (end 163.966667 119.92) (width 0.5) (layer "B.Cu") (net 9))
 (segment (start 164.96 109) (end 164.96 118.926667) (width 0.5) (layer "B.Cu") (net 9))
 (segment (start 172.185 116.735) (end 169 119.92) (width 0.5) (layer "B.Cu") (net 2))
 (segment (start 172.185 109) (end 172.185 116.735) (width 0.5) (layer "B.Cu") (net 2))
 (segment (start 179.185 109) (end 179.185 114.701667) (width 0.5) (layer "B.Cu") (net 20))
 (segment (start 179.185 114.701667) (end 173.966667 119.92) (width 0.5) (layer "B.Cu") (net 20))
 (segment (start 150 106.5) (end 152 106.5) (width 0.5) (layer "B.Cu") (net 7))
 (segment (start 154 104.5) (end 165.5 104.5) (width 0.5) (layer "B.Cu") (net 7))
 (segment (start 152 106.5) (end 154 104.5) (width 0.5) (layer "B.Cu") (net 7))
 (segment (start 167.5 106.5) (end 167.5 109) (width 0.5) (layer "B.Cu") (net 7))
 (segment (start 142.82 106.705) (end 149.795 106.705) (width 0.5) (layer "B.Cu") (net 7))
 (segment (start 149.795 106.705) (end 150 106.5) (width 0.5) (layer "B.Cu") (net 7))
 (segment (start 165.5 104.5) (end 167.5 106.5) (width 0.5) (layer "B.Cu") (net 7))
 (segment (start 143.025 106.5) (end 142.82 106.705) (width 0.5) (layer "B.Cu") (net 7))
 (segment (start 150 101) (end 151.5 99.5) (width 0.5) (layer "B.Cu") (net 8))
 (segment (start 180.5 99.5) (end 181.725 100.725) (width 0.5) (layer "B.Cu") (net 8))
 (segment (start 181.725 100.725) (end 181.725 109) (width 0.5) (layer "B.Cu") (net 8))
 (segment (start 150 101.5) (end 150 101) (width 0.5) (layer "B.Cu") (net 8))
 (segment (start 149.875 101.625) (end 150 101.5) (width 0.5) (layer "B.Cu") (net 8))
 (segment (start 142.945 101.5) (end 142.82 101.625) (width 0.5) (layer "B.Cu") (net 8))
 (segment (start 151.5 99.5) (end 180.5 99.5) (width 0.5) (layer "B.Cu") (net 8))
 (segment (start 142.82 101.625) (end 149.875 101.625) (width 0.5) (layer "B.Cu") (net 8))
 (segment (start 150 104) (end 151.5 104) (width 0.5) (layer "B.Cu") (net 1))
 (segment (start 151.5 104) (end 153.5 102) (width 0.5) (layer "B.Cu") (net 1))
 (segment (start 174.725 104.225) (end 174.725 109) (width 0.5) (layer "B.Cu") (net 1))
 (segment (start 149.835 104.165) (end 150 104) (width 0.5) (layer "B.Cu") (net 1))
 (segment (start 142.985 104) (end 142.82 104.165) (width 0.5) (layer "B.Cu") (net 1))
 (segment (start 150.066667 103.933333) (end 150 104) (width 0.5) (layer "B.Cu") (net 1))
 (segment (start 172.5 102) (end 174.725 104.225) (width 0.5) (layer "B.Cu") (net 1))
 (segment (start 153.5 102) (end 172.5 102) (width 0.5) (layer "B.Cu") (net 1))
 (segment (start 142.82 104.165) (end 149.835 104.165) (width 0.5) (layer "B.Cu") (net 1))
 (segment (start 150 109) (end 152.5 109) (width 0.5) (layer "B.Cu") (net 3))
 (segment (start 143.065 109) (end 142.82 109.245) (width 0.5) (layer "B.Cu") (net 3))
 (segment (start 158 106.5) (end 160.5 109) (width 0.5) (layer "B.Cu") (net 3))
 (segment (start 149.755 109.245) (end 150 109) (width 0.5) (layer "B.Cu") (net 3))
 (segment (start 155 106.5) (end 158 106.5) (width 0.5) (layer "B.Cu") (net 3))
 (segment (start 142.82 109.245) (end 149.755 109.245) (width 0.5) (layer "B.Cu") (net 3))
 (segment (start 152.5 109) (end 155 106.5) (width 0.5) (layer "B.Cu") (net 3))
 (segment (start 135.145 101.68) (end 135.2 101.625) (width 0.5) (layer "B.Cu") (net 10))
 (segment (start 129.5 101.68) (end 135.145 101.68) (width 0.5) (layer "B.Cu") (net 10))
 (segment (start 135.145 109.3) (end 135.2 109.245) (width 0.5) (layer "B.Cu") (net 13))
 (segment (start 129.5 109.3) (end 135.145 109.3) (width 0.5) (layer "B.Cu") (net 13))
 (segment (start 135.145 106.76) (end 135.2 106.705) (width 0.5) (layer "B.Cu") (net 12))
 (segment (start 129.5 106.76) (end 135.145 106.76) (width 0.5) (layer "B.Cu") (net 12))
 (segment (start 135.145 104.22) (end 135.2 104.165) (width 0.5) (layer "B.Cu") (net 11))
 (segment (start 129.5 104.22) (end 135.145 104.22) (width 0.5) (layer "B.Cu") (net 11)))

